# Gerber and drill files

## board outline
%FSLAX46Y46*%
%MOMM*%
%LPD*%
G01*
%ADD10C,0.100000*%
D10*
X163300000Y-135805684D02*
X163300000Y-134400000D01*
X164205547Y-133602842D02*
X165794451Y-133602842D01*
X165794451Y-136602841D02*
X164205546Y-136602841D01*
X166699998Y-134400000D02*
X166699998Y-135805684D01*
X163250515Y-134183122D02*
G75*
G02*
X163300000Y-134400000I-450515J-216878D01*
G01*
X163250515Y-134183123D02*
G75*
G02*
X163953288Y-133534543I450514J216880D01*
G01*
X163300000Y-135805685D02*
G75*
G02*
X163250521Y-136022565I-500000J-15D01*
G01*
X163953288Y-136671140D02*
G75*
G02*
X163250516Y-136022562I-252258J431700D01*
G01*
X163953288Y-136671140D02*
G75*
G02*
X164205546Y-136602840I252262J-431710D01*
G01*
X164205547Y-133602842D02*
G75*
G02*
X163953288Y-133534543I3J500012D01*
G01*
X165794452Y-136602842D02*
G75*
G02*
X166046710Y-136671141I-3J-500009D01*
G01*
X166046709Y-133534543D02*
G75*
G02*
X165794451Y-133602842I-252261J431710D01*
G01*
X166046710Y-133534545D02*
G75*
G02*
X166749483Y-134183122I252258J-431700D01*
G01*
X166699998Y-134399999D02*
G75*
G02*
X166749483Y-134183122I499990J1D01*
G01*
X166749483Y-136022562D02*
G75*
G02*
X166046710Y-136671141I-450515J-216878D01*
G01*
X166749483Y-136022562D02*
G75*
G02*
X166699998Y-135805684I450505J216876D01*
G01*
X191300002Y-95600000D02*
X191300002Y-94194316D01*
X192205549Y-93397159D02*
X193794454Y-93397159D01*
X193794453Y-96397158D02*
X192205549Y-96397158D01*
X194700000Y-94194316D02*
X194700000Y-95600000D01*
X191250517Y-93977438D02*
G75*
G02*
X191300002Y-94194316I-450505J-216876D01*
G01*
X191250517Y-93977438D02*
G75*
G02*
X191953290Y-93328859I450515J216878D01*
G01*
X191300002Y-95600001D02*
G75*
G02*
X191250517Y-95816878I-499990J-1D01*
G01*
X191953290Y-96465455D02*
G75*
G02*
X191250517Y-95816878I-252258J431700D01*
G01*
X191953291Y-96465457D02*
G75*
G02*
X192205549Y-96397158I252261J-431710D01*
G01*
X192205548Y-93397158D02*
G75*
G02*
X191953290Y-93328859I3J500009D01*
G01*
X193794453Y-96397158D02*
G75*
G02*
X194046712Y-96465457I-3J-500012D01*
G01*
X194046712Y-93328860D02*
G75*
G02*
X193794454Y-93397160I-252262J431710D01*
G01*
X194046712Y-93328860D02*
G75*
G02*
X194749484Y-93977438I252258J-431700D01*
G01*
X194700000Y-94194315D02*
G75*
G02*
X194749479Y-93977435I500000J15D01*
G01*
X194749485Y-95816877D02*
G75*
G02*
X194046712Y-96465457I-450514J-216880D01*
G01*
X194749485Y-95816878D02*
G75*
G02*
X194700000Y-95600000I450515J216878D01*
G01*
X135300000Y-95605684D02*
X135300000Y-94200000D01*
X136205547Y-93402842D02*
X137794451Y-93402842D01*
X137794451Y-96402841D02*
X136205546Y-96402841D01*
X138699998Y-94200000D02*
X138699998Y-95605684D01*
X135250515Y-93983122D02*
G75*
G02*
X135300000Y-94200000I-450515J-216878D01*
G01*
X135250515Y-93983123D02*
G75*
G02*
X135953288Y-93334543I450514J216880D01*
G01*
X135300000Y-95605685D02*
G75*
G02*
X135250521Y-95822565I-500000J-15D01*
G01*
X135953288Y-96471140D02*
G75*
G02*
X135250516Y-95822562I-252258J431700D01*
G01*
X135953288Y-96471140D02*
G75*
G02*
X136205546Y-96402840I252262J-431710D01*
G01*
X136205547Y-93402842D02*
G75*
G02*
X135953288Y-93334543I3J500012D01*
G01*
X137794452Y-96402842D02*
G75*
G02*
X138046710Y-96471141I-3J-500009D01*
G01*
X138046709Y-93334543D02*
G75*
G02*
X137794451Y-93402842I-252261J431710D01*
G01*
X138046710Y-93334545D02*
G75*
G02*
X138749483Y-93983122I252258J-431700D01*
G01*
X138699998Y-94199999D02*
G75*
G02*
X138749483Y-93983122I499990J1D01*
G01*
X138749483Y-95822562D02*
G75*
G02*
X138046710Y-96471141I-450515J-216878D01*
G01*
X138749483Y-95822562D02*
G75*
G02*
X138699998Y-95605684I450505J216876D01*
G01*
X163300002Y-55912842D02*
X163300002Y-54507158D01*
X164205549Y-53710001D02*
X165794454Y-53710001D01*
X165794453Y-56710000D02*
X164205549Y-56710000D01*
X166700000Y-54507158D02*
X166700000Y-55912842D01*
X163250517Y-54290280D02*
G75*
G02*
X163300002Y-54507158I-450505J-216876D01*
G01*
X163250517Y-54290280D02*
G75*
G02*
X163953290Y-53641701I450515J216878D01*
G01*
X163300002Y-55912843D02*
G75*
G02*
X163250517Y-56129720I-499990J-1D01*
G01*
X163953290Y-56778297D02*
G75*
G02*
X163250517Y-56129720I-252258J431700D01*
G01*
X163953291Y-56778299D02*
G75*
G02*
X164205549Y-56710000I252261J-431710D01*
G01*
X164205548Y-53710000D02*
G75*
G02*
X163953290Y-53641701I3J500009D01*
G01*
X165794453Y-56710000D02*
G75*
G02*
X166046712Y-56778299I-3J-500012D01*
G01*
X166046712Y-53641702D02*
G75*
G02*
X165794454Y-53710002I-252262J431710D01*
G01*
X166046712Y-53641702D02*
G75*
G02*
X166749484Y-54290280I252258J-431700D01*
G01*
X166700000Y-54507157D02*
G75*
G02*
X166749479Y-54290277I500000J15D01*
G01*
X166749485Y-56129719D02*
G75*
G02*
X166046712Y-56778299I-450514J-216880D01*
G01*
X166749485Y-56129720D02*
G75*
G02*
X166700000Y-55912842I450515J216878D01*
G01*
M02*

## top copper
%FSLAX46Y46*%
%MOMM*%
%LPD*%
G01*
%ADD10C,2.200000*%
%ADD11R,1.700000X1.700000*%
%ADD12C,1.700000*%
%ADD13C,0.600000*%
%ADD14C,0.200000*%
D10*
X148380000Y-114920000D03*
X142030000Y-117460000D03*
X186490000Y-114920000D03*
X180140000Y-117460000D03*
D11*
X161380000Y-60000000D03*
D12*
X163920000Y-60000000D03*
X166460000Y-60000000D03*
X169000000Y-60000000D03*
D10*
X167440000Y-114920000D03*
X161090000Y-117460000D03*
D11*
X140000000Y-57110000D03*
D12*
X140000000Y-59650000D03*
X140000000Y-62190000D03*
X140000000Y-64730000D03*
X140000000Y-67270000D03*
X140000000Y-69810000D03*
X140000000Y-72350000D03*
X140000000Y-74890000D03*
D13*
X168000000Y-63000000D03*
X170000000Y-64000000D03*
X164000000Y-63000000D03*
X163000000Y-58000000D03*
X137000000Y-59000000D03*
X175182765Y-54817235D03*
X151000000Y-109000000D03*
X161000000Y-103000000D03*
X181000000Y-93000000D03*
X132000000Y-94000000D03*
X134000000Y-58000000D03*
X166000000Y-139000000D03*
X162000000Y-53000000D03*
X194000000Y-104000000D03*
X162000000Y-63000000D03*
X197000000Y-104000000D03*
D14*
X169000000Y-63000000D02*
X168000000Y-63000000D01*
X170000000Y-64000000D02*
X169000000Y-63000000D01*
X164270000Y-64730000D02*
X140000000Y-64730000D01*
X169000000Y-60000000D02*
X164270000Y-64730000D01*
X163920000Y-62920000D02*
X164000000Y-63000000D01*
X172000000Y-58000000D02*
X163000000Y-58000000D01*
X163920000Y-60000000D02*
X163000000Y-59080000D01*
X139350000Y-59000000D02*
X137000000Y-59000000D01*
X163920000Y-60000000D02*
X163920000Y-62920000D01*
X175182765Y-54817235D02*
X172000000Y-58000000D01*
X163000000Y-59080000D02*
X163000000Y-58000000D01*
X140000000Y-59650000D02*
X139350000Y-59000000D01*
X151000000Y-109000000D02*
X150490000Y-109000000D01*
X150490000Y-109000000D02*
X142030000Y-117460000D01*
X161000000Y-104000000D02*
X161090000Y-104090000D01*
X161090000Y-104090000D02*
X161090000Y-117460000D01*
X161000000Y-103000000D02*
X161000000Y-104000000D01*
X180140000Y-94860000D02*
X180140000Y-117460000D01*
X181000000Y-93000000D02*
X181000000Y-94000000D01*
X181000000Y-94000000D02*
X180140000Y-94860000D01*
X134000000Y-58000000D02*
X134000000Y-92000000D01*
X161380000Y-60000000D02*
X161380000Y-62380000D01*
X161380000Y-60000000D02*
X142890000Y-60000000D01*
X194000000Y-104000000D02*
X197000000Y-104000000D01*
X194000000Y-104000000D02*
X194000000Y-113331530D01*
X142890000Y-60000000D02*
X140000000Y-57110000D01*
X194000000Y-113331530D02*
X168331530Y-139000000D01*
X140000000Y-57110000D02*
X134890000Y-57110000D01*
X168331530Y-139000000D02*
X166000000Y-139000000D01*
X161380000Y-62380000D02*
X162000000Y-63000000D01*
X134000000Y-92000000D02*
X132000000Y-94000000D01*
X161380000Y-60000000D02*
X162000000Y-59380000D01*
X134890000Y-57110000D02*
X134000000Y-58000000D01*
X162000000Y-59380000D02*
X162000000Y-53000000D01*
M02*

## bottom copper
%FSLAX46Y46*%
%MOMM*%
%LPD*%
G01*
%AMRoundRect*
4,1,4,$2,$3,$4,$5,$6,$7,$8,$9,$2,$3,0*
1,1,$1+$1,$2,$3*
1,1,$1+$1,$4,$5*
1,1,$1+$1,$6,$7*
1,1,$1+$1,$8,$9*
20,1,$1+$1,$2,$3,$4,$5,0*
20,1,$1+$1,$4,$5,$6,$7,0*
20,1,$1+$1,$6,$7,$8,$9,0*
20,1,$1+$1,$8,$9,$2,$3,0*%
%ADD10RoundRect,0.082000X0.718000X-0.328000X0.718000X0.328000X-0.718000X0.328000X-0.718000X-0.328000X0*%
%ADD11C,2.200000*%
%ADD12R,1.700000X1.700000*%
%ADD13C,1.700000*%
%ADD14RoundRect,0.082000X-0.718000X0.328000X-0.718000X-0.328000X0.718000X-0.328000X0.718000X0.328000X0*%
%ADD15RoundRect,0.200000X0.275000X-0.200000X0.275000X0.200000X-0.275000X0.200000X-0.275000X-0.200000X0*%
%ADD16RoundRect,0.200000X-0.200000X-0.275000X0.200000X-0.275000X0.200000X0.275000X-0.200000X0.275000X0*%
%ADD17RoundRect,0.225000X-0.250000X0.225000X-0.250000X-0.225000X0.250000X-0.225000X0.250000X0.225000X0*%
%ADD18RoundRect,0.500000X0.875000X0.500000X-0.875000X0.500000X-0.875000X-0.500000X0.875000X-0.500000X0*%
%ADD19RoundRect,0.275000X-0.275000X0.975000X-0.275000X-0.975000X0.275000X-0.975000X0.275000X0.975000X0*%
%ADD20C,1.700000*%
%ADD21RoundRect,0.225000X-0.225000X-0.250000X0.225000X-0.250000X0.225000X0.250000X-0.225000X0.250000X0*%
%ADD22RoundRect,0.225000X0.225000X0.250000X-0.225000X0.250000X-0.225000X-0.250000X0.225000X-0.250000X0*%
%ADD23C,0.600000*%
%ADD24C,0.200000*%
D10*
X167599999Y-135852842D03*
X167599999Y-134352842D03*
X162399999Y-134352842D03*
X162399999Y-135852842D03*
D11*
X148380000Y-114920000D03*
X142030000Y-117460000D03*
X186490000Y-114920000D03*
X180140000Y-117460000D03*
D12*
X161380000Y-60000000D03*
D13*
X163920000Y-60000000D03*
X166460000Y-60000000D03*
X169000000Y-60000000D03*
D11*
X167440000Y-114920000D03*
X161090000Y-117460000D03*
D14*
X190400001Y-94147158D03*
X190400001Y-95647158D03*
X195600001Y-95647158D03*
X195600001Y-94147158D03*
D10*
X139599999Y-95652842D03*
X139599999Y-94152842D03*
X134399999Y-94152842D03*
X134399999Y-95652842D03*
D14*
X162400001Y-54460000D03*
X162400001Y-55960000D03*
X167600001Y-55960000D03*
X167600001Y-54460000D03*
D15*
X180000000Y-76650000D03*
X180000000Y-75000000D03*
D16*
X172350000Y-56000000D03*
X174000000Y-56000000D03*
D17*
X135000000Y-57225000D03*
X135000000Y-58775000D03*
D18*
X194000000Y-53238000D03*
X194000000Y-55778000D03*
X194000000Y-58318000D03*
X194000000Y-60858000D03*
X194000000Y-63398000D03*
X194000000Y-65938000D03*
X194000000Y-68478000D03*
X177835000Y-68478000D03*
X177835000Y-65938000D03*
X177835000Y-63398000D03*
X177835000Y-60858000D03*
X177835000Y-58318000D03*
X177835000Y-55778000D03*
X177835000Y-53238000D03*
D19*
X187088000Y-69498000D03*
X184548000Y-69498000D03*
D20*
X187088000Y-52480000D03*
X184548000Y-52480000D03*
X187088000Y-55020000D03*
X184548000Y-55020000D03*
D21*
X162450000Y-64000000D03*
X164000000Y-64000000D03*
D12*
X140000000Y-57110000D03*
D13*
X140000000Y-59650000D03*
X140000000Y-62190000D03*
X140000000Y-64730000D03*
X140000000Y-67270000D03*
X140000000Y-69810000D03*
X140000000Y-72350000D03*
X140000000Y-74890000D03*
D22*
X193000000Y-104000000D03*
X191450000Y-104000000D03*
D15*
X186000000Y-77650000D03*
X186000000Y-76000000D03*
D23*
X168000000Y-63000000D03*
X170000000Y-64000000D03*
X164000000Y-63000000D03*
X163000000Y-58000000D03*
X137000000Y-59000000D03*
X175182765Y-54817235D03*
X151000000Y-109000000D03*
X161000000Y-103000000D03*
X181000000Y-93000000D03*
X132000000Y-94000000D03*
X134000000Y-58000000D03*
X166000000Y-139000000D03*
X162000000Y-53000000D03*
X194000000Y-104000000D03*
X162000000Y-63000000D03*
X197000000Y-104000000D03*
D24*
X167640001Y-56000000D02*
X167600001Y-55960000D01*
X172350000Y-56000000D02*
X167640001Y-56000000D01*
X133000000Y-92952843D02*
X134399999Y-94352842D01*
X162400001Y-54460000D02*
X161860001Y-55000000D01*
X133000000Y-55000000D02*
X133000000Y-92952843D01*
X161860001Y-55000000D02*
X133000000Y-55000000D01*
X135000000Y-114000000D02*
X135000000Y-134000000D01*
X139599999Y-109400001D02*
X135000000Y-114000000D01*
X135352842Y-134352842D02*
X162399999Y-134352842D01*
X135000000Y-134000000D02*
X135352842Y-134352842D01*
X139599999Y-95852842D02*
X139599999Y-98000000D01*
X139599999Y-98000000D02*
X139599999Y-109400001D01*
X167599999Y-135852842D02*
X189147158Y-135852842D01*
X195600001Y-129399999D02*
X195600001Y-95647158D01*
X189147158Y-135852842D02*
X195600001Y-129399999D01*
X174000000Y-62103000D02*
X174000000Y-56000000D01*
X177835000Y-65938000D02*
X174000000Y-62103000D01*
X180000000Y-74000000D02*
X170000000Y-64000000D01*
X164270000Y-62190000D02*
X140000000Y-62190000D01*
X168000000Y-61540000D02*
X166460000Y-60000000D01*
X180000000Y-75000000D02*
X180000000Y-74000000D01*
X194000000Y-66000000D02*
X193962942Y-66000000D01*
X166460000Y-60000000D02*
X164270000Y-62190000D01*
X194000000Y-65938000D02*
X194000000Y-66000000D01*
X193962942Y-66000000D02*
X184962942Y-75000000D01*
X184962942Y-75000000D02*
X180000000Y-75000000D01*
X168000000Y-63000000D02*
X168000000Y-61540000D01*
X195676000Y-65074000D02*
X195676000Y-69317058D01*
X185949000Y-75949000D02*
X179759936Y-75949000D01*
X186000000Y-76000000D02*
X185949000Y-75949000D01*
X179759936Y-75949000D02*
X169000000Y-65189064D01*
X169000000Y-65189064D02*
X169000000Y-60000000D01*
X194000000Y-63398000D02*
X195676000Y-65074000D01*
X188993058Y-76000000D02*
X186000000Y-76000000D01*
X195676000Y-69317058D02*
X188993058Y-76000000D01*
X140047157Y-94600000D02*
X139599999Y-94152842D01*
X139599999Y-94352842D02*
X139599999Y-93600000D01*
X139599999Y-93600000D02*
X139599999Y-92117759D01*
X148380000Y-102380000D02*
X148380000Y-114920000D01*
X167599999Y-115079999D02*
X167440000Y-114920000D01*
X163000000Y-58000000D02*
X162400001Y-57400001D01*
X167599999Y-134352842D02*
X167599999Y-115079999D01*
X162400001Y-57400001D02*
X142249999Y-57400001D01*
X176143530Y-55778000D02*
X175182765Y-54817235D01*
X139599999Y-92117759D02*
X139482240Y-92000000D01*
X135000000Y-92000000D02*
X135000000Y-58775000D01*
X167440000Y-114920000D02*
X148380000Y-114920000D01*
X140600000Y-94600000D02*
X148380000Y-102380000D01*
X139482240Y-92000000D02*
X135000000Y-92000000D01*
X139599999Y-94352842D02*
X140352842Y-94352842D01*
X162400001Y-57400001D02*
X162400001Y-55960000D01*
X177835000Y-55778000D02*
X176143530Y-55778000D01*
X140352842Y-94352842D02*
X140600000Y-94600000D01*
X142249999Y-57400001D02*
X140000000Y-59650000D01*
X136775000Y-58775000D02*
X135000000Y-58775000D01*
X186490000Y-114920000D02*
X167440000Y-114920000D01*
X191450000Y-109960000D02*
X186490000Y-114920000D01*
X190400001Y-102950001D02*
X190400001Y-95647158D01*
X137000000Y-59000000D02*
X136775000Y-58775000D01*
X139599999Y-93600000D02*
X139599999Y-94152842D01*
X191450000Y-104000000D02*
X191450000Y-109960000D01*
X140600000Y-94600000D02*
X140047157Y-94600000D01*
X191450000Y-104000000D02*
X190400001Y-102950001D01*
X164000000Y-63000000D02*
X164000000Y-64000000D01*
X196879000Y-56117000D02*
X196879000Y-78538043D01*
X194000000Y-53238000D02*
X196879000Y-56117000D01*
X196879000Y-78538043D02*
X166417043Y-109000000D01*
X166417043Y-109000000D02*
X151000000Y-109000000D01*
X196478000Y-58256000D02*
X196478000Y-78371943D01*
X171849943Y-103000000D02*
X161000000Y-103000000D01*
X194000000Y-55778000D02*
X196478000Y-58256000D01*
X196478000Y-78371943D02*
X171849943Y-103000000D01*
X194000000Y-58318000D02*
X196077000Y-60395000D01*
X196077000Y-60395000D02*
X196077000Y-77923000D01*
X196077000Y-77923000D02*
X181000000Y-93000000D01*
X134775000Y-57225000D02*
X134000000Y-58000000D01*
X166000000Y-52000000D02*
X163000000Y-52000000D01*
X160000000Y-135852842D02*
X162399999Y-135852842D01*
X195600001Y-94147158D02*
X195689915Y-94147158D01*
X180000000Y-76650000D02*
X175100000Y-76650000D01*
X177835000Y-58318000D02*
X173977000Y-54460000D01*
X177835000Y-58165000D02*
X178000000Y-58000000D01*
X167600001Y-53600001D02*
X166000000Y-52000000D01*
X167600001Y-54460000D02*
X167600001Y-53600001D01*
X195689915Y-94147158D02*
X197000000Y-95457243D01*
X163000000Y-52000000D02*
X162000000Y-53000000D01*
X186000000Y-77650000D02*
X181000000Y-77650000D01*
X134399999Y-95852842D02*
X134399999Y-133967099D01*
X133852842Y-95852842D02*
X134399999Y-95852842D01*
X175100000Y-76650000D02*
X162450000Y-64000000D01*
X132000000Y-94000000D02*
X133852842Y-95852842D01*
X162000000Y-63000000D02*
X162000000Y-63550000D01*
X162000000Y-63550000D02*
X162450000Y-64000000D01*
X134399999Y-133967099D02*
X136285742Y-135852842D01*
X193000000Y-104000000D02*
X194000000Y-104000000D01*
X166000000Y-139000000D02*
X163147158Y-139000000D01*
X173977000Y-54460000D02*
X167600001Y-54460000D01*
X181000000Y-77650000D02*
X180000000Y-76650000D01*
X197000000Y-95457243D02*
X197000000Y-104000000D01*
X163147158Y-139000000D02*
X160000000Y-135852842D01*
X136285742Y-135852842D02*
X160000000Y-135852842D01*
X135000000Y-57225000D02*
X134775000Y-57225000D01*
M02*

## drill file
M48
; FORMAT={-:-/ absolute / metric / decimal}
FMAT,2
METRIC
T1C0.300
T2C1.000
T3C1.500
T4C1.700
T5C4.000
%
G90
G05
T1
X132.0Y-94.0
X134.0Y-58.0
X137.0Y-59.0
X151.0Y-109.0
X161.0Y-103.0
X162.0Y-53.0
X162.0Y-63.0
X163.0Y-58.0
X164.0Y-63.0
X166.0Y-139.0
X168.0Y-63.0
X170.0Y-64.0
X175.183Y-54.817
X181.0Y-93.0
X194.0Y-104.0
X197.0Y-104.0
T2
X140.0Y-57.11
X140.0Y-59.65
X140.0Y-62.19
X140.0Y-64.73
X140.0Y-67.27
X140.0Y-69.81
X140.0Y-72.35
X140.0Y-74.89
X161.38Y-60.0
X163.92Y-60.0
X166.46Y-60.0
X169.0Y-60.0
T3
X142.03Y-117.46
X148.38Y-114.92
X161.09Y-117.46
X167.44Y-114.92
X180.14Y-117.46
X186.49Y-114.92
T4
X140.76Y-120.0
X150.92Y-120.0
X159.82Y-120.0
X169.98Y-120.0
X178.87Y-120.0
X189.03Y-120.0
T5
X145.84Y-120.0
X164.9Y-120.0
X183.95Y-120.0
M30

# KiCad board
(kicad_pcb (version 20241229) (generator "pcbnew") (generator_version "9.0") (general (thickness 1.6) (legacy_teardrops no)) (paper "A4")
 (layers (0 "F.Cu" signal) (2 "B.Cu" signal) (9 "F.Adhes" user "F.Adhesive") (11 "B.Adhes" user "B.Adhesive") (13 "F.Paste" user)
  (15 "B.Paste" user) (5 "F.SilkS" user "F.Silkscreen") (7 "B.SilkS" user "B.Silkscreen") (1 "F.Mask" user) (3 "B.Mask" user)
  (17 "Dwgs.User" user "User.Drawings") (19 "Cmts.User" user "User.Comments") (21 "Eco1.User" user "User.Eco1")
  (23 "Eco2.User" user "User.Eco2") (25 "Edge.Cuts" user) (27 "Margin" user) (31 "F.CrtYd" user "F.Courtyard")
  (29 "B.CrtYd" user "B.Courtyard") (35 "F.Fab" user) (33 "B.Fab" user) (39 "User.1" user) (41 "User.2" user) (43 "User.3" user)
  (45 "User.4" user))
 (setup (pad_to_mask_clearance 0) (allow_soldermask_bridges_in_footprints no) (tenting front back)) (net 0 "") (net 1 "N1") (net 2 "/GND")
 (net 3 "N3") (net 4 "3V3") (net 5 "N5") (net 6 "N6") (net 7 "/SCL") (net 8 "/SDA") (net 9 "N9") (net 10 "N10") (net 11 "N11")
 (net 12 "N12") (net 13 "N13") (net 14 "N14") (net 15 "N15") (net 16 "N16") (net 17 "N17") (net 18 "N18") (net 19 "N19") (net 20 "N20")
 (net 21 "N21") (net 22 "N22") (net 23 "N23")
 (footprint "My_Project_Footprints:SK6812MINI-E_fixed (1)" (layer "F.Cu") (at 165 135 180)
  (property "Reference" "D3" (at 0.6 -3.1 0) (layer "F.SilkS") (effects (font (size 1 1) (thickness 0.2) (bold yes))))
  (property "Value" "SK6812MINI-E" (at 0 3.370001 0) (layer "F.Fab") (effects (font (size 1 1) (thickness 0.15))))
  (fp_line (start 1.7 -0.805684) (end 1.7 0.6) (stroke (width 0.1) (type solid)) (layer "Edge.Cuts"))
  (fp_line (start 0.794453 1.397158) (end -0.794451 1.397158) (stroke (width 0.1) (type solid)) (layer "Edge.Cuts"))
  (fp_line (start -0.794451 -1.602841) (end 0.794454 -1.602841) (stroke (width 0.1) (type solid)) (layer "Edge.Cuts"))
  (fp_line (start -1.699998 0.6) (end -1.699998 -0.805684) (stroke (width 0.1) (type solid)) (layer "Edge.Cuts"))
  (fp_arc (start 1.749485 0.816878) (mid 1.712528 0.711226) (end 1.7 0.6) (stroke (width 0.1) (type solid)) (layer "Edge.Cuts"))
  (fp_arc (start 1.749485 0.816877) (mid 1.638073 1.401193) (end 1.046712 1.465457) (stroke (width 0.1) (type solid)) (layer "Edge.Cuts"))
  (fp_arc (start 1.7 -0.805685) (mid 1.712528 -0.91691) (end 1.749485 -1.022562) (stroke (width 0.1) (type solid)) (layer "Edge.Cuts"))
  (fp_arc (start 1.046712 -1.67114) (mid 1.638072 -1.606876) (end 1.749485 -1.022562) (stroke (width 0.1) (type solid)) (layer "Edge.Cuts"))
  (fp_arc (start 1.046712 -1.67114) (mid 0.925124 -1.620218) (end 0.794454 -1.602841) (stroke (width 0.1) (type solid)) (layer "Edge.Cuts"))
  (fp_arc (start 0.794453 1.397158) (mid 0.925124 1.414535) (end 1.046712 1.465457) (stroke (width 0.1) (type solid)) (layer "Edge.Cuts"))
  (fp_arc (start -0.794452 -1.602842) (mid -0.925122 -1.620219) (end -1.04671 -1.671141) (stroke (width 0.1) (type solid))
   (layer "Edge.Cuts"))
  (fp_arc (start -1.046709 1.465457) (mid -0.925121 1.414535) (end -0.794451 1.397158) (stroke (width 0.1) (type solid)) (layer "Edge.Cuts"))
  (fp_arc (start -1.04671 1.465455) (mid -1.638069 1.401192) (end -1.749483 0.816878) (stroke (width 0.1) (type solid)) (layer "Edge.Cuts"))
  (fp_arc (start -1.699998 0.600001) (mid -1.712526 0.711226) (end -1.749483 0.816878) (stroke (width 0.1) (type solid)) (layer "Edge.Cuts"))
  (fp_arc (start -1.749483 -1.022562) (mid -1.63807 -1.606877) (end -1.04671 -1.671141) (stroke (width 0.1) (type solid))
   (layer "Edge.Cuts"))
  (fp_arc (start -1.749483 -1.022562) (mid -1.712526 -0.91691) (end -1.699998 -0.805684) (stroke (width 0.1) (type solid))
   (layer "Edge.Cuts"))
  (pad "1" smd roundrect (at -2.599999 -0.852842 90) (size 0.82 1.6) (layers "B.Cu" "B.Mask" "B.Paste") (roundrect_rratio 0.1) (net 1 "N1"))
  (pad "2" smd roundrect (at -2.599999 0.647158 90) (size 0.82 1.6) (layers "B.Cu" "B.Mask" "B.Paste") (roundrect_rratio 0.1) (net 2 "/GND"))
  (pad "3" smd roundrect (at 2.600001 0.647158 90) (size 0.82 1.6) (layers "B.Cu" "B.Mask" "B.Paste") (roundrect_rratio 0.1) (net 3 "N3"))
  (pad "4" smd roundrect (at 2.600001 -0.852842 90) (size 0.82 1.6) (layers "B.Cu" "B.Mask" "B.Paste") (roundrect_rratio 0.1) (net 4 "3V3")))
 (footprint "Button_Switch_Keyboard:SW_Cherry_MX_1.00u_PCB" (layer "F.Cu") (at 148.38 114.92)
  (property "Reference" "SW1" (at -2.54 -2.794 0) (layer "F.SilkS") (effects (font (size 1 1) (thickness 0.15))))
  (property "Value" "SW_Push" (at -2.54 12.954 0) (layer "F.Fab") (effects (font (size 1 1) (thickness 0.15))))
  (pad "" np_thru_hole circle (at -7.62 5.08) (size 1.7 1.7) (drill 1.7) (layers "*.Cu" "*.Mask"))
  (pad "" np_thru_hole circle (at -2.54 5.08) (size 4 4) (drill 4) (layers "*.Cu" "*.Mask"))
  (pad "" np_thru_hole circle (at 2.54 5.08) (size 1.7 1.7) (drill 1.7) (layers "*.Cu" "*.Mask"))
  (pad "1" thru_hole circle (at 0 0) (size 2.2 2.2) (drill 1.5) (layers "*.Cu" "*.Mask") (remove_unused_layers no) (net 2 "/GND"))
  (pad "2" thru_hole circle (at -6.35 2.54) (size 2.2 2.2) (drill 1.5) (layers "*.Cu" "*.Mask") (remove_unused_layers no) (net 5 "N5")))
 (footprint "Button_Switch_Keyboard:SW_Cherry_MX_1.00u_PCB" (layer "F.Cu") (at 186.49 114.92)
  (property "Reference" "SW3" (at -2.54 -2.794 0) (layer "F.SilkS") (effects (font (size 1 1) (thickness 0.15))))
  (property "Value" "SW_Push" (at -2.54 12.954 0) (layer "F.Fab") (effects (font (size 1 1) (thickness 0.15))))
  (pad "" np_thru_hole circle (at -7.62 5.08) (size 1.7 1.7) (drill 1.7) (layers "*.Cu" "*.Mask"))
  (pad "" np_thru_hole circle (at -2.54 5.08) (size 4 4) (drill 4) (layers "*.Cu" "*.Mask"))
  (pad "" np_thru_hole circle (at 2.54 5.08) (size 1.7 1.7) (drill 1.7) (layers "*.Cu" "*.Mask"))
  (pad "1" thru_hole circle (at 0 0) (size 2.2 2.2) (drill 1.5) (layers "*.Cu" "*.Mask") (remove_unused_layers no) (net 2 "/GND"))
  (pad "2" thru_hole circle (at -6.35 2.54) (size 2.2 2.2) (drill 1.5) (layers "*.Cu" "*.Mask") (remove_unused_layers no) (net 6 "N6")))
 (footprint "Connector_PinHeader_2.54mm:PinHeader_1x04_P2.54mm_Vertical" (layer "F.Cu") (at 161.38 60 90)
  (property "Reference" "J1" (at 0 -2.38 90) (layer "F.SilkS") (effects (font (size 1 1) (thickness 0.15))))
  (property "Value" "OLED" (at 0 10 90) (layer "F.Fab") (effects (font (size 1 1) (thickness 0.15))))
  (pad "1" thru_hole rect (at 0 0 90) (size 1.7 1.7) (drill 1) (layers "*.Cu" "*.Mask") (remove_unused_layers no) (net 4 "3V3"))
  (pad "2" thru_hole circle (at 0 2.54 90) (size 1.7 1.7) (drill 1) (layers "*.Cu" "*.Mask") (remove_unused_layers no) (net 2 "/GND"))
  (pad "3" thru_hole circle (at 0 5.08 90) (size 1.7 1.7) (drill 1) (layers "*.Cu" "*.Mask") (remove_unused_layers no) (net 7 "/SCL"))
  (pad "4" thru_hole circle (at 0 7.62 90) (size 1.7 1.7) (drill 1) (layers "*.Cu" "*.Mask") (remove_unused_layers no) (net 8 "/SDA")))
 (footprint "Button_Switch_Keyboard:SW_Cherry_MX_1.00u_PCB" (layer "F.Cu") (at 167.44 114.92)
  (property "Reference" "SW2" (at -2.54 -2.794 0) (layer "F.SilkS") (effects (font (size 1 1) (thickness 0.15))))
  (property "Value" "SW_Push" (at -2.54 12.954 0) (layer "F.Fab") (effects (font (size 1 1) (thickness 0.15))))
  (pad "" np_thru_hole circle (at -7.62 5.08) (size 1.7 1.7) (drill 1.7) (layers "*.Cu" "*.Mask"))
  (pad "" np_thru_hole circle (at -2.54 5.08) (size 4 4) (drill 4) (layers "*.Cu" "*.Mask"))
  (pad "" np_thru_hole circle (at 2.54 5.08) (size 1.7 1.7) (drill 1.7) (layers "*.Cu" "*.Mask"))
  (pad "1" thru_hole circle (at 0 0) (size 2.2 2.2) (drill 1.5) (layers "*.Cu" "*.Mask") (remove_unused_layers no) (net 2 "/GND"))
  (pad "2" thru_hole circle (at -6.35 2.54) (size 2.2 2.2) (drill 1.5) (layers "*.Cu" "*.Mask") (remove_unused_layers no) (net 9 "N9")))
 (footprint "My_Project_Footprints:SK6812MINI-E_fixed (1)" (layer "F.Cu") (at 193 95)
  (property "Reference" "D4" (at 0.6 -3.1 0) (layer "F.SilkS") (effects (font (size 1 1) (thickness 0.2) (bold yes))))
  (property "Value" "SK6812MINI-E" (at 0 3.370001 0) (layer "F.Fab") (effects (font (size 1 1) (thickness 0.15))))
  (fp_line (start -1.699998 0.6) (end -1.699998 -0.805684) (stroke (width 0.1) (type solid)) (layer "Edge.Cuts"))
  (fp_line (start -0.794451 -1.602841) (end 0.794454 -1.602841) (stroke (width 0.1) (type solid)) (layer "Edge.Cuts"))
  (fp_line (start 0.794453 1.397158) (end -0.794451 1.397158) (stroke (width 0.1) (type solid)) (layer "Edge.Cuts"))
  (fp_line (start 1.7 -0.805684) (end 1.7 0.6) (stroke (width 0.1) (type solid)) (layer "Edge.Cuts"))
  (fp_arc (start -1.749483 -1.022562) (mid -1.712526 -0.91691) (end -1.699998 -0.805684) (stroke (width 0.1) (type solid))
   (layer "Edge.Cuts"))
  (fp_arc (start -1.749483 -1.022562) (mid -1.63807 -1.606877) (end -1.04671 -1.671141) (stroke (width 0.1) (type solid))
   (layer "Edge.Cuts"))
  (fp_arc (start -1.699998 0.600001) (mid -1.712526 0.711226) (end -1.749483 0.816878) (stroke (width 0.1) (type solid)) (layer "Edge.Cuts"))
  (fp_arc (start -1.04671 1.465455) (mid -1.638069 1.401192) (end -1.749483 0.816878) (stroke (width 0.1) (type solid)) (layer "Edge.Cuts"))
  (fp_arc (start -1.046709 1.465457) (mid -0.925121 1.414535) (end -0.794451 1.397158) (stroke (width 0.1) (type solid)) (layer "Edge.Cuts"))
  (fp_arc (start -0.794452 -1.602842) (mid -0.925122 -1.620219) (end -1.04671 -1.671141) (stroke (width 0.1) (type solid))
   (layer "Edge.Cuts"))
  (fp_arc (start 0.794453 1.397158) (mid 0.925124 1.414535) (end 1.046712 1.465457) (stroke (width 0.1) (type solid)) (layer "Edge.Cuts"))
  (fp_arc (start 1.046712 -1.67114) (mid 0.925124 -1.620218) (end 0.794454 -1.602841) (stroke (width 0.1) (type solid)) (layer "Edge.Cuts"))
  (fp_arc (start 1.046712 -1.67114) (mid 1.638072 -1.606876) (end 1.749485 -1.022562) (stroke (width 0.1) (type solid)) (layer "Edge.Cuts"))
  (fp_arc (start 1.7 -0.805685) (mid 1.712528 -0.91691) (end 1.749485 -1.022562) (stroke (width 0.1) (type solid)) (layer "Edge.Cuts"))
  (fp_arc (start 1.749485 0.816877) (mid 1.638073 1.401193) (end 1.046712 1.465457) (stroke (width 0.1) (type solid)) (layer "Edge.Cuts"))
  (fp_arc (start 1.749485 0.816878) (mid 1.712528 0.711226) (end 1.7 0.6) (stroke (width 0.1) (type solid)) (layer "Edge.Cuts"))
  (pad "1" smd roundrect (at -2.599999 -0.852842 270) (size 0.82 1.6) (layers "B.Cu" "B.Mask" "B.Paste") (roundrect_rratio 0.1)
   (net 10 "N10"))
  (pad "2" smd roundrect (at -2.599999 0.647158 270) (size 0.82 1.6) (layers "B.Cu" "B.Mask" "B.Paste") (roundrect_rratio 0.1)
   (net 2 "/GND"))
  (pad "3" smd roundrect (at 2.600001 0.647158 270) (size 0.82 1.6) (layers "B.Cu" "B.Mask" "B.Paste") (roundrect_rratio 0.1) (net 1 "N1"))
  (pad "4" smd roundrect (at 2.600001 -0.852842 270) (size 0.82 1.6) (layers "B.Cu" "B.Mask" "B.Paste") (roundrect_rratio 0.1) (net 4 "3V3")))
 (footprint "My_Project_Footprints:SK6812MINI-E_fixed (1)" (layer "F.Cu") (at 137 94.8 180)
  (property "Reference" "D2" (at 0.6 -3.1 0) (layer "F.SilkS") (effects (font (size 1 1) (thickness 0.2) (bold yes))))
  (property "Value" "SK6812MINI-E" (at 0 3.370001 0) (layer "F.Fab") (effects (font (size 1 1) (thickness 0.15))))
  (fp_line (start 1.7 -0.805684) (end 1.7 0.6) (stroke (width 0.1) (type solid)) (layer "Edge.Cuts"))
  (fp_line (start 0.794453 1.397158) (end -0.794451 1.397158) (stroke (width 0.1) (type solid)) (layer "Edge.Cuts"))
  (fp_line (start -0.794451 -1.602841) (end 0.794454 -1.602841) (stroke (width 0.1) (type solid)) (layer "Edge.Cuts"))
  (fp_line (start -1.699998 0.6) (end -1.699998 -0.805684) (stroke (width 0.1) (type solid)) (layer "Edge.Cuts"))
  (fp_arc (start 1.749485 0.816878) (mid 1.712528 0.711226) (end 1.7 0.6) (stroke (width 0.1) (type solid)) (layer "Edge.Cuts"))
  (fp_arc (start 1.749485 0.816877) (mid 1.638073 1.401193) (end 1.046712 1.465457) (stroke (width 0.1) (type solid)) (layer "Edge.Cuts"))
  (fp_arc (start 1.7 -0.805685) (mid 1.712528 -0.91691) (end 1.749485 -1.022562) (stroke (width 0.1) (type solid)) (layer "Edge.Cuts"))
  (fp_arc (start 1.046712 -1.67114) (mid 1.638072 -1.606876) (end 1.749485 -1.022562) (stroke (width 0.1) (type solid)) (layer "Edge.Cuts"))
  (fp_arc (start 1.046712 -1.67114) (mid 0.925124 -1.620218) (end 0.794454 -1.602841) (stroke (width 0.1) (type solid)) (layer "Edge.Cuts"))
  (fp_arc (start 0.794453 1.397158) (mid 0.925124 1.414535) (end 1.046712 1.465457) (stroke (width 0.1) (type solid)) (layer "Edge.Cuts"))
  (fp_arc (start -0.794452 -1.602842) (mid -0.925122 -1.620219) (end -1.04671 -1.671141) (stroke (width 0.1) (type solid))
   (layer "Edge.Cuts"))
  (fp_arc (start -1.046709 1.465457) (mid -0.925121 1.414535) (end -0.794451 1.397158) (stroke (width 0.1) (type solid)) (layer "Edge.Cuts"))
  (fp_arc (start -1.04671 1.465455) (mid -1.638069 1.401192) (end -1.749483 0.816878) (stroke (width 0.1) (type solid)) (layer "Edge.Cuts"))
  (fp_arc (start -1.699998 0.600001) (mid -1.712526 0.711226) (end -1.749483 0.816878) (stroke (width 0.1) (type solid)) (layer "Edge.Cuts"))
  (fp_arc (start -1.749483 -1.022562) (mid -1.63807 -1.606877) (end -1.04671 -1.671141) (stroke (width 0.1) (type solid))
   (layer "Edge.Cuts"))
  (fp_arc (start -1.749483 -1.022562) (mid -1.712526 -0.91691) (end -1.699998 -0.805684) (stroke (width 0.1) (type solid))
   (layer "Edge.Cuts"))
  (pad "1" smd roundrect (at -2.599999 -0.852842 90) (size 0.82 1.6) (layers "B.Cu" "B.Mask" "B.Paste") (roundrect_rratio 0.1) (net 3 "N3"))
  (pad "2" smd roundrect (at -2.599999 0.647158 90) (size 0.82 1.6) (layers "B.Cu" "B.Mask" "B.Paste") (roundrect_rratio 0.1) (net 2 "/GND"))
  (pad "3" smd roundrect (at 2.600001 0.647158 90) (size 0.82 1.6) (layers "B.Cu" "B.Mask" "B.Paste") (roundrect_rratio 0.1) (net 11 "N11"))
  (pad "4" smd roundrect (at 2.600001 -0.852842 90) (size 0.82 1.6) (layers "B.Cu" "B.Mask" "B.Paste") (roundrect_rratio 0.1) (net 4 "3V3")))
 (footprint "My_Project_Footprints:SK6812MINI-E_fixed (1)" (layer "F.Cu") (at 165 55.312842)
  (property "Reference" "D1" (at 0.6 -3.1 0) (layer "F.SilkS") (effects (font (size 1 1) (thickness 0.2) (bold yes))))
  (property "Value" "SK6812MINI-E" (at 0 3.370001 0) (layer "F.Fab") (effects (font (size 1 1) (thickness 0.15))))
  (fp_line (start -1.699998 0.6) (end -1.699998 -0.805684) (stroke (width 0.1) (type solid)) (layer "Edge.Cuts"))
  (fp_line (start -0.794451 -1.602841) (end 0.794454 -1.602841) (stroke (width 0.1) (type solid)) (layer "Edge.Cuts"))
  (fp_line (start 0.794453 1.397158) (end -0.794451 1.397158) (stroke (width 0.1) (type solid)) (layer "Edge.Cuts"))
  (fp_line (start 1.7 -0.805684) (end 1.7 0.6) (stroke (width 0.1) (type solid)) (layer "Edge.Cuts"))
  (fp_arc (start -1.749483 -1.022562) (mid -1.712526 -0.91691) (end -1.699998 -0.805684) (stroke (width 0.1) (type solid))
   (layer "Edge.Cuts"))
  (fp_arc (start -1.749483 -1.022562) (mid -1.63807 -1.606877) (end -1.04671 -1.671141) (stroke (width 0.1) (type solid))
   (layer "Edge.Cuts"))
  (fp_arc (start -1.699998 0.600001) (mid -1.712526 0.711226) (end -1.749483 0.816878) (stroke (width 0.1) (type solid)) (layer "Edge.Cuts"))
  (fp_arc (start -1.04671 1.465455) (mid -1.638069 1.401192) (end -1.749483 0.816878) (stroke (width 0.1) (type solid)) (layer "Edge.Cuts"))
  (fp_arc (start -1.046709 1.465457) (mid -0.925121 1.414535) (end -0.794451 1.397158) (stroke (width 0.1) (type solid)) (layer "Edge.Cuts"))
  (fp_arc (start -0.794452 -1.602842) (mid -0.925122 -1.620219) (end -1.04671 -1.671141) (stroke (width 0.1) (type solid))
   (layer "Edge.Cuts"))
  (fp_arc (start 0.794453 1.397158) (mid 0.925124 1.414535) (end 1.046712 1.465457) (stroke (width 0.1) (type solid)) (layer "Edge.Cuts"))
  (fp_arc (start 1.046712 -1.67114) (mid 0.925124 -1.620218) (end 0.794454 -1.602841) (stroke (width 0.1) (type solid)) (layer "Edge.Cuts"))
  (fp_arc (start 1.046712 -1.67114) (mid 1.638072 -1.606876) (end 1.749485 -1.022562) (stroke (width 0.1) (type solid)) (layer "Edge.Cuts"))
  (fp_arc (start 1.7 -0.805685) (mid 1.712528 -0.91691) (end 1.749485 -1.022562) (stroke (width 0.1) (type solid)) (layer "Edge.Cuts"))
  (fp_arc (start 1.749485 0.816877) (mid 1.638073 1.401193) (end 1.046712 1.465457) (stroke (width 0.1) (type solid)) (layer "Edge.Cuts"))
  (fp_arc (start 1.749485 0.816878) (mid 1.712528 0.711226) (end 1.7 0.6) (stroke (width 0.1) (type solid)) (layer "Edge.Cuts"))
  (pad "1" smd roundrect (at -2.599999 -0.852842 270) (size 0.82 1.6) (layers "B.Cu" "B.Mask" "B.Paste") (roundrect_rratio 0.1)
   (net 11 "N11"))
  (pad "2" smd roundrect (at -2.599999 0.647158 270) (size 0.82 1.6) (layers "B.Cu" "B.Mask" "B.Paste") (roundrect_rratio 0.1)
   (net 2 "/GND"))
  (pad "3" smd roundrect (at 2.600001 0.647158 270) (size 0.82 1.6) (layers "B.Cu" "B.Mask" "B.Paste") (roundrect_rratio 0.1) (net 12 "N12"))
  (pad "4" smd roundrect (at 2.600001 -0.852842 270) (size 0.82 1.6) (layers "B.Cu" "B.Mask" "B.Paste") (roundrect_rratio 0.1) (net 4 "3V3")))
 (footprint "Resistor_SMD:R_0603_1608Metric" (layer "B.Cu") (at 180 75.825 90)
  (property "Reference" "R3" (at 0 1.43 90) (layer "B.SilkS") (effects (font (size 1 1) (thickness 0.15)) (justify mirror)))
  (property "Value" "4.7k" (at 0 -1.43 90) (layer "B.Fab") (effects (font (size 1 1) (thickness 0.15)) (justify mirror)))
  (pad "1" smd roundrect (at -0.825 0 90) (size 0.8 0.95) (layers "B.Cu" "B.Mask" "B.Paste") (roundrect_rratio 0.25) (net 4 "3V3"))
  (pad "2" smd roundrect (at 0.825 0 90) (size 0.8 0.95) (layers "B.Cu" "B.Mask" "B.Paste") (roundrect_rratio 0.25) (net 7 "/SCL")))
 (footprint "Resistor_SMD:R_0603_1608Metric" (layer "B.Cu") (at 173.175 56)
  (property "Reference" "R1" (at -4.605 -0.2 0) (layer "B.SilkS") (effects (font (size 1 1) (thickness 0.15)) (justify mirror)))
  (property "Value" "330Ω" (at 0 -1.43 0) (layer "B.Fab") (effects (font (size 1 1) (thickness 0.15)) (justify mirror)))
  (pad "1" smd roundrect (at -0.825 0) (size 0.8 0.95) (layers "B.Cu" "B.Mask" "B.Paste") (roundrect_rratio 0.25) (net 12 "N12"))
  (pad "2" smd roundrect (at 0.825 0) (size 0.8 0.95) (layers "B.Cu" "B.Mask" "B.Paste") (roundrect_rratio 0.25) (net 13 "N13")))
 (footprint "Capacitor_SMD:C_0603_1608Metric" (layer "B.Cu") (at 135 58 -90)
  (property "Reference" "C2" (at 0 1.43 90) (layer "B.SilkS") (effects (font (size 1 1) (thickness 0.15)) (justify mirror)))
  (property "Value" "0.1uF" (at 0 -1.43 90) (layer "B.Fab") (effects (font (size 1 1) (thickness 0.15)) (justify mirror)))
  (pad "1" smd roundrect (at -0.775 0 270) (size 0.9 0.95) (layers "B.Cu" "B.Mask" "B.Paste") (roundrect_rratio 0.25) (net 4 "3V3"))
  (pad "2" smd roundrect (at 0.775 0 270) (size 0.9 0.95) (layers "B.Cu" "B.Mask" "B.Paste") (roundrect_rratio 0.25) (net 2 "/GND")))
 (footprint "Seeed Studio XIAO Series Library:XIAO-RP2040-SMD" (layer "B.Cu") (at 186 60.858 180)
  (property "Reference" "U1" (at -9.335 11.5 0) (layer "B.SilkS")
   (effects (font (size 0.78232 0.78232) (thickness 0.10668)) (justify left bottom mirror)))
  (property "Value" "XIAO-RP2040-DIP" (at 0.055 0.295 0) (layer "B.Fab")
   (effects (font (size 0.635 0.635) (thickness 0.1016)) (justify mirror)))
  (pad "1" smd roundrect (at -8 7.62 180) (size 2.75 2) (layers "B.Cu" "B.Mask" "B.Paste") (roundrect_rratio 0.25) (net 5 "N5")
   (solder_mask_margin 0.0508) (thermal_bridge_angle 45))
  (pad "2" smd roundrect (at -8 5.08 180) (size 2.75 2) (layers "B.Cu" "B.Mask" "B.Paste") (roundrect_rratio 0.25) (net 9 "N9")
   (solder_mask_margin 0.0508) (thermal_bridge_angle 45))
  (pad "3" smd roundrect (at -8 2.54 180) (size 2.75 2) (layers "B.Cu" "B.Mask" "B.Paste") (roundrect_rratio 0.25) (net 6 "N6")
   (solder_mask_margin 0.0508) (thermal_bridge_angle 45))
  (pad "4" smd roundrect (at -8 0 180) (size 2.75 2) (layers "B.Cu" "B.Mask" "B.Paste") (roundrect_rratio 0.25) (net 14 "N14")
   (solder_mask_margin 0.0508) (thermal_bridge_angle 45))
  (pad "5" smd roundrect (at -8 -2.54 180) (size 2.75 2) (layers "B.Cu" "B.Mask" "B.Paste") (roundrect_rratio 0.25) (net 8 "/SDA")
   (solder_mask_margin 0.0508) (thermal_bridge_angle 45))
  (pad "6" smd roundrect (at -8 -5.08 180) (size 2.75 2) (layers "B.Cu" "B.Mask" "B.Paste") (roundrect_rratio 0.25) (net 7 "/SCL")
   (solder_mask_margin 0.0508) (thermal_bridge_angle 45))
  (pad "7" smd roundrect (at -8 -7.62 180) (size 2.75 2) (layers "B.Cu" "B.Mask" "B.Paste") (roundrect_rratio 0.25) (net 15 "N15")
   (solder_mask_margin 0.0508) (thermal_bridge_angle 45))
  (pad "8" smd roundrect (at 8.165 -7.62 180) (size 2.75 2) (layers "B.Cu" "B.Mask" "B.Paste") (roundrect_rratio 0.25) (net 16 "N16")
   (solder_mask_margin 0.0508) (thermal_bridge_angle 45))
  (pad "9" smd roundrect (at 8.165 -5.08 180) (size 2.75 2) (layers "B.Cu" "B.Mask" "B.Paste") (roundrect_rratio 0.25) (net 13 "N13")
   (solder_mask_margin 0.0508) (thermal_bridge_angle 45))
  (pad "10" smd roundrect (at 8.165 -2.54 180) (size 2.75 2) (layers "B.Cu" "B.Mask" "B.Paste") (roundrect_rratio 0.25) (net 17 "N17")
   (solder_mask_margin 0.0508) (thermal_bridge_angle 45))
  (pad "11" smd roundrect (at 8.165 0 180) (size 2.75 2) (layers "B.Cu" "B.Mask" "B.Paste") (roundrect_rratio 0.25) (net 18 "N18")
   (solder_mask_margin 0.0508) (thermal_bridge_angle 45))
  (pad "12" smd roundrect (at 8.165 2.54 180) (size 2.75 2) (layers "B.Cu" "B.Mask" "B.Paste") (roundrect_rratio 0.25) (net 4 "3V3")
   (solder_mask_margin 0.0508) (thermal_bridge_angle 45))
  (pad "13" smd roundrect (at 8.165 5.08 180) (size 2.75 2) (layers "B.Cu" "B.Mask" "B.Paste") (roundrect_rratio 0.25) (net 2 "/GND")
   (solder_mask_margin 0.0508) (thermal_bridge_angle 45))
  (pad "14" smd roundrect (at 8.165 7.62 180) (size 2.75 2) (layers "B.Cu" "B.Mask" "B.Paste") (roundrect_rratio 0.25) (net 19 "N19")
   (solder_mask_margin 0.0508) (thermal_bridge_angle 45))
  (pad "15" smd roundrect (at -1.088 -8.64 270) (size 2.5 1.1) (layers "B.Cu" "B.Mask" "B.Paste") (roundrect_rratio 0.25)
   (thermal_bridge_angle 45))
  (pad "16" smd roundrect (at 1.452 -8.64 270) (size 2.5 1.1) (layers "B.Cu" "B.Mask" "B.Paste") (roundrect_rratio 0.25)
   (thermal_bridge_angle 45))
  (pad "17" smd circle (at -1.088 8.378 180) (size 1.7 1.7) (layers "B.Cu" "B.Mask" "B.Paste"))
  (pad "18" smd circle (at 1.452 8.378 180) (size 1.7 1.7) (layers "B.Cu" "B.Mask" "B.Paste"))
  (pad "19" smd circle (at -1.088 5.838 180) (size 1.7 1.7) (layers "B.Cu" "B.Mask" "B.Paste"))
  (pad "20" smd circle (at 1.452 5.838 180) (size 1.7 1.7) (layers "B.Cu" "B.Mask" "B.Paste")))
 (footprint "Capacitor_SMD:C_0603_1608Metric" (layer "B.Cu") (at 163.225 64)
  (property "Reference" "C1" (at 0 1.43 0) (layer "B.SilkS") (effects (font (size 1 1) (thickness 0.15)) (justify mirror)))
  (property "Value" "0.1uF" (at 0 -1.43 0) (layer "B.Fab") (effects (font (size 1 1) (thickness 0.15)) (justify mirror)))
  (pad "1" smd roundrect (at -0.775 0) (size 0.9 0.95) (layers "B.Cu" "B.Mask" "B.Paste") (roundrect_rratio 0.25) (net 4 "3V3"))
  (pad "2" smd roundrect (at 0.775 0) (size 0.9 0.95) (layers "B.Cu" "B.Mask" "B.Paste") (roundrect_rratio 0.25) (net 2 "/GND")))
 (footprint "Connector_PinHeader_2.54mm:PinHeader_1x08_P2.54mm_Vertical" (layer "B.Cu") (at 140 57.11 180)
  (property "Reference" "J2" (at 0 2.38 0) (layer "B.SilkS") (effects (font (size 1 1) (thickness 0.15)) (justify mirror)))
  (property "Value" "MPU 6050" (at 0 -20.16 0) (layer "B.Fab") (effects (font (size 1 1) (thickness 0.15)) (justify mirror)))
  (pad "1" thru_hole rect (at 0 0 180) (size 1.7 1.7) (drill 1) (layers "*.Cu" "*.Mask") (remove_unused_layers no) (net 4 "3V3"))
  (pad "2" thru_hole circle (at 0 -2.54 180) (size 1.7 1.7) (drill 1) (layers "*.Cu" "*.Mask") (remove_unused_layers no) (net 2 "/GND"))
  (pad "3" thru_hole circle (at 0 -5.08 180) (size 1.7 1.7) (drill 1) (layers "*.Cu" "*.Mask") (remove_unused_layers no) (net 7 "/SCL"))
  (pad "4" thru_hole circle (at 0 -7.62 180) (size 1.7 1.7) (drill 1) (layers "*.Cu" "*.Mask") (remove_unused_layers no) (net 8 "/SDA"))
  (pad "5" thru_hole circle (at 0 -10.16 180) (size 1.7 1.7) (drill 1) (layers "*.Cu" "*.Mask") (remove_unused_layers no) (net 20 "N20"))
  (pad "6" thru_hole circle (at 0 -12.7 180) (size 1.7 1.7) (drill 1) (layers "*.Cu" "*.Mask") (remove_unused_layers no) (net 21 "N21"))
  (pad "7" thru_hole circle (at 0 -15.24 180) (size 1.7 1.7) (drill 1) (layers "*.Cu" "*.Mask") (remove_unused_layers no) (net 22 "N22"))
  (pad "8" thru_hole circle (at 0 -17.78 180) (size 1.7 1.7) (drill 1) (layers "*.Cu" "*.Mask") (remove_unused_layers no) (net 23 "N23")))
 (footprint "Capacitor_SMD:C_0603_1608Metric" (layer "B.Cu") (at 192.225 104 180)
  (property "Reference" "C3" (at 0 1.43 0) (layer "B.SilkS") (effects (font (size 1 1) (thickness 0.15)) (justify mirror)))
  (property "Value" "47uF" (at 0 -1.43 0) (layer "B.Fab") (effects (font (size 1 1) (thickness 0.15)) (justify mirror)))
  (pad "1" smd roundrect (at -0.775 0 180) (size 0.9 0.95) (layers "B.Cu" "B.Mask" "B.Paste") (roundrect_rratio 0.25) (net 4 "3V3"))
  (pad "2" smd roundrect (at 0.775 0 180) (size 0.9 0.95) (layers "B.Cu" "B.Mask" "B.Paste") (roundrect_rratio 0.25) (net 2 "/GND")))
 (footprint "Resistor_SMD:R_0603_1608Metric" (layer "B.Cu") (at 186 76.825 90)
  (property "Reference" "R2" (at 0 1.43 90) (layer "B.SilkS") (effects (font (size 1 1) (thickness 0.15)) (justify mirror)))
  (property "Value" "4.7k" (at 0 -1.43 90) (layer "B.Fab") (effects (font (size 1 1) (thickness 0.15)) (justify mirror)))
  (pad "1" smd roundrect (at -0.825 0 90) (size 0.8 0.95) (layers "B.Cu" "B.Mask" "B.Paste") (roundrect_rratio 0.25) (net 4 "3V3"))
  (pad "2" smd roundrect (at 0.825 0 90) (size 0.8 0.95) (layers "B.Cu" "B.Mask" "B.Paste") (roundrect_rratio 0.25) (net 8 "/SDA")))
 (segment (start 167.640001 56) (end 167.600001 55.96) (width 0.2) (layer "B.Cu") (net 12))
 (segment (start 172.35 56) (end 167.640001 56) (width 0.2) (layer "B.Cu") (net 12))
 (segment (start 133 92.952843) (end 134.399999 94.352842) (width 0.2) (layer "B.Cu") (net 11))
 (segment (start 162.400001 54.46) (end 161.860001 55) (width 0.2) (layer "B.Cu") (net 11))
 (segment (start 133 55) (end 133 92.952843) (width 0.2) (layer "B.Cu") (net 11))
 (segment (start 161.860001 55) (end 133 55) (width 0.2) (layer "B.Cu") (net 11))
 (segment (start 135 114) (end 135 134) (width 0.2) (layer "B.Cu") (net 3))
 (segment (start 139.599999 109.400001) (end 135 114) (width 0.2) (layer "B.Cu") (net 3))
 (segment (start 135.352842 134.352842) (end 162.399999 134.352842) (width 0.2) (layer "B.Cu") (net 3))
 (segment (start 135 134) (end 135.352842 134.352842) (width 0.2) (layer "B.Cu") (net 3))
 (segment (start 139.599999 95.852842) (end 139.599999 98) (width 0.2) (layer "B.Cu") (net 3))
 (segment (start 139.599999 98) (end 139.599999 109.400001) (width 0.2) (layer "B.Cu") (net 3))
 (segment (start 167.599999 135.852842) (end 189.147158 135.852842) (width 0.2) (layer "B.Cu") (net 1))
 (segment (start 195.600001 129.399999) (end 195.600001 95.647158) (width 0.2) (layer "B.Cu") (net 1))
 (segment (start 189.147158 135.852842) (end 195.600001 129.399999) (width 0.2) (layer "B.Cu") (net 1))
 (segment (start 174 62.103) (end 174 56) (width 0.2) (layer "B.Cu") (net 13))
 (segment (start 177.835 65.938) (end 174 62.103) (width 0.2) (layer "B.Cu") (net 13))
 (segment (start 169 63) (end 168 63) (width 0.2) (layer "F.Cu") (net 7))
 (segment (start 170 64) (end 169 63) (width 0.2) (layer "F.Cu") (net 7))
 (via (at 168 63) (size 0.6) (drill 0.3) (layers "F.Cu" "B.Cu") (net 7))
 (via (at 170 64) (size 0.6) (drill 0.3) (layers "F.Cu" "B.Cu") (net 7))
 (segment (start 180 74) (end 170 64) (width 0.2) (layer "B.Cu") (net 7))
 (segment (start 164.27 62.19) (end 140 62.19) (width 0.2) (layer "B.Cu") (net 7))
 (segment (start 168 61.54) (end 166.46 60) (width 0.2) (layer "B.Cu") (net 7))
 (segment (start 180 75) (end 180 74) (width 0.2) (layer "B.Cu") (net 7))
 (segment (start 194 66) (end 193.962942 66) (width 0.2) (layer "B.Cu") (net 7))
 (segment (start 166.46 60) (end 164.27 62.19) (width 0.2) (layer "B.Cu") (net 7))
 (segment (start 194 65.938) (end 194 66) (width 0.2) (layer "B.Cu") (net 7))
 (segment (start 193.962942 66) (end 184.962942 75) (width 0.2) (layer "B.Cu") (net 7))
 (segment (start 184.962942 75) (end 180 75) (width 0.2) (layer "B.Cu") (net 7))
 (segment (start 168 63) (end 168 61.54) (width 0.2) (layer "B.Cu") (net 7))
 (segment (start 164.27 64.73) (end 140 64.73) (width 0.2) (layer "F.Cu") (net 8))
 (segment (start 169 60) (end 164.27 64.73) (width 0.2) (layer "F.Cu") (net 8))
 (segment (start 195.676 65.074) (end 195.676 69.317058) (width 0.2) (layer "B.Cu") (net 8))
 (segment (start 185.949 75.949) (end 179.759936 75.949) (width 0.2) (layer "B.Cu") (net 8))
 (segment (start 186 76) (end 185.949 75.949) (width 0.2) (layer "B.Cu") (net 8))
 (segment (start 179.759936 75.949) (end 169 65.189064) (width 0.2) (layer "B.Cu") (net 8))
 (segment (start 169 65.189064) (end 169 60) (width 0.2) (layer "B.Cu") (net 8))
 (segment (start 194 63.398) (end 195.676 65.074) (width 0.2) (layer "B.Cu") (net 8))
 (segment (start 188.993058 76) (end 186 76) (width 0.2) (layer "B.Cu") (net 8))
 (segment (start 195.676 69.317058) (end 188.993058 76) (width 0.2) (layer "B.Cu") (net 8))
 (segment (start 163.92 62.92) (end 164 63) (width 0.2) (layer "F.Cu") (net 2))
 (segment (start 172 58) (end 163 58) (width 0.2) (layer "F.Cu") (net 2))
 (segment (start 163.92 60) (end 163 59.08) (width 0.2) (layer "F.Cu") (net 2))
 (segment (start 139.35 59) (end 137 59) (width 0.2) (layer "F.Cu") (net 2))
 (segment (start 163.92 60) (end 163.92 62.92) (width 0.2) (layer "F.Cu") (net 2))
 (segment (start 175.182765 54.817235) (end 172 58) (width 0.2) (layer "F.Cu") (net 2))
 (segment (start 163 59.08) (end 163 58) (width 0.2) (layer "F.Cu") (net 2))
 (segment (start 140 59.65) (end 139.35 59) (width 0.2) (layer "F.Cu") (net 2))
 (via (at 164 63) (size 0.6) (drill 0.3) (layers "F.Cu" "B.Cu") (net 2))
 (via (at 163 58) (size 0.6) (drill 0.3) (layers "F.Cu" "B.Cu") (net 2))
 (via (at 137 59) (size 0.6) (drill 0.3) (layers "F.Cu" "B.Cu") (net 2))
 (via (at 175.182765 54.817235) (size 0.6) (drill 0.3) (layers "F.Cu" "B.Cu") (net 2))
 (segment (start 140.047157 94.6) (end 139.599999 94.152842) (width 0.2) (layer "B.Cu") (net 2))
 (segment (start 139.599999 94.352842) (end 139.599999 93.6) (width 0.2) (layer "B.Cu") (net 2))
 (segment (start 139.599999 93.6) (end 139.599999 92.117759) (width 0.2) (layer "B.Cu") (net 2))
 (segment (start 148.38 102.38) (end 148.38 114.92) (width 0.2) (layer "B.Cu") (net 2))
 (segment (start 167.599999 115.079999) (end 167.44 114.92) (width 0.2) (layer "B.Cu") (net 2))
 (segment (start 163 58) (end 162.400001 57.400001) (width 0.2) (layer "B.Cu") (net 2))
 (segment (start 167.599999 134.352842) (end 167.599999 115.079999) (width 0.2) (layer "B.Cu") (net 2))
 (segment (start 162.400001 57.400001) (end 142.249999 57.400001) (width 0.2) (layer "B.Cu") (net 2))
 (segment (start 176.14353 55.778) (end 175.182765 54.817235) (width 0.2) (layer "B.Cu") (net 2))
 (segment (start 139.599999 92.117759) (end 139.48224 92) (width 0.2) (layer "B.Cu") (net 2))
 (segment (start 135 92) (end 135 58.775) (width 0.2) (layer "B.Cu") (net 2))
 (segment (start 167.44 114.92) (end 148.38 114.92) (width 0.2) (layer "B.Cu") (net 2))
 (segment (start 140.6 94.6) (end 148.38 102.38) (width 0.2) (layer "B.Cu") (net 2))
 (segment (start 139.48224 92) (end 135 92) (width 0.2) (layer "B.Cu") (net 2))
 (segment (start 139.599999 94.352842) (end 140.352842 94.352842) (width 0.2) (layer "B.Cu") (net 2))
 (segment (start 162.400001 57.400001) (end 162.400001 55.96) (width 0.2) (layer "B.Cu") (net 2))
 (segment (start 177.835 55.778) (end 176.14353 55.778) (width 0.2) (layer "B.Cu") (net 2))
 (segment (start 140.352842 94.352842) (end 140.6 94.6) (width 0.2) (layer "B.Cu") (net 2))
 (segment (start 142.249999 57.400001) (end 140 59.65) (width 0.2) (layer "B.Cu") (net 2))
 (segment (start 136.775 58.775) (end 135 58.775) (width 0.2) (layer "B.Cu") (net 2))
 (segment (start 186.49 114.92) (end 167.44 114.92) (width 0.2) (layer "B.Cu") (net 2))
 (segment (start 191.45 109.96) (end 186.49 114.92) (width 0.2) (layer "B.Cu") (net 2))
 (segment (start 190.400001 102.950001) (end 190.400001 95.647158) (width 0.2) (layer "B.Cu") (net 2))
 (segment (start 137 59) (end 136.775 58.775) (width 0.2) (layer "B.Cu") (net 2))
 (segment (start 139.599999 93.6) (end 139.599999 94.152842) (width 0.2) (layer "B.Cu") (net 2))
 (segment (start 191.45 104) (end 191.45 109.96) (width 0.2) (layer "B.Cu") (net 2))
 (segment (start 140.6 94.6) (end 140.047157 94.6) (width 0.2) (layer "B.Cu") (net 2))
 (segment (start 191.45 104) (end 190.400001 102.950001) (width 0.2) (layer "B.Cu") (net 2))
 (segment (start 164 63) (end 164 64) (width 0.2) (layer "B.Cu") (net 2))
 (segment (start 151 109) (end 150.49 109) (width 0.2) (layer "F.Cu") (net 5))
 (segment (start 150.49 109) (end 142.03 117.46) (width 0.2) (layer "F.Cu") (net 5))
 (via (at 151 109) (size 0.6) (drill 0.3) (layers "F.Cu" "B.Cu") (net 5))
 (segment (start 196.879 56.117) (end 196.879 78.538043) (width 0.2) (layer "B.Cu") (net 5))
 (segment (start 194 53.238) (end 196.879 56.117) (width 0.2) (layer "B.Cu") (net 5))
 (segment (start 196.879 78.538043) (end 166.417043 109) (width 0.2) (layer "B.Cu") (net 5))
 (segment (start 166.417043 109) (end 151 109) (width 0.2) (layer "B.Cu") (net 5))
 (segment (start 161 104) (end 161.09 104.09) (width 0.2) (layer "F.Cu") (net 9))
 (segment (start 161.09 104.09) (end 161.09 117.46) (width 0.2) (layer "F.Cu") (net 9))
 (segment (start 161 103) (end 161 104) (width 0.2) (layer "F.Cu") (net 9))
 (via (at 161 103) (size 0.6) (drill 0.3) (layers "F.Cu" "B.Cu") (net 9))
 (segment (start 196.478 58.256) (end 196.478 78.371943) (width 0.2) (layer "B.Cu") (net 9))
 (segment (start 171.849943 103) (end 161 103) (width 0.2) (layer "B.Cu") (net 9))
 (segment (start 194 55.778) (end 196.478 58.256) (width 0.2) (layer "B.Cu") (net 9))
 (segment (start 196.478 78.371943) (end 171.849943 103) (width 0.2) (layer "B.Cu") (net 9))
 (segment (start 180.14 94.86) (end 180.14 117.46) (width 0.2) (layer "F.Cu") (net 6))
 (segment (start 181 93) (end 181 94) (width 0.2) (layer "F.Cu") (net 6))
 (segment (start 181 94) (end 180.14 94.86) (width 0.2) (layer "F.Cu") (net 6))
 (via (at 181 93) (size 0.6) (drill 0.3) (layers "F.Cu" "B.Cu") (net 6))
 (segment (start 194 58.318) (end 196.077 60.395) (width 0.2) (layer "B.Cu") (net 6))
 (segment (start 196.077 60.395) (end 196.077 77.923) (width 0.2) (layer "B.Cu") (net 6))
 (segment (start 196.077 77.923) (end 181 93) (width 0.2) (layer "B.Cu") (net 6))
 (segment (start 134 58) (end 134 92) (width 0.2) (layer "F.Cu") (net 4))
 (segment (start 161.38 60) (end 161.38 62.38) (width 0.2) (layer "F.Cu") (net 4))
 (segment (start 161.38 60) (end 142.89 60) (width 0.2) (layer "F.Cu") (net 4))
 (segment (start 194 104) (end 197 104) (width 0.2) (layer "F.Cu") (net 4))
 (segment (start 194 104) (end 194 113.33153) (width 0.2) (layer "F.Cu") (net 4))
 (segment (start 142.89 60) (end 140 57.11) (width 0.2) (layer "F.Cu") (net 4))
 (segment (start 194 113.33153) (end 168.33153 139) (width 0.2) (layer "F.Cu") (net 4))
 (segment (start 140 57.11) (end 134.89 57.11) (width 0.2) (layer "F.Cu") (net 4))
 (segment (start 168.33153 139) (end 166 139) (width 0.2) (layer "F.Cu") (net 4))
 (segment (start 161.38 62.38) (end 162 63) (width 0.2) (layer "F.Cu") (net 4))
 (segment (start 134 92) (end 132 94) (width 0.2) (layer "F.Cu") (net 4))
 (segment (start 161.38 60) (end 162 59.38) (width 0.2) (layer "F.Cu") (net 4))
 (segment (start 134.89 57.11) (end 134 58) (width 0.2) (layer "F.Cu") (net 4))
 (segment (start 162 59.38) (end 162 53) (width 0.2) (layer "F.Cu") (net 4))
 (via (at 132 94) (size 0.6) (drill 0.3) (layers "F.Cu" "B.Cu") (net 4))
 (via (at 134 58) (size 0.6) (drill 0.3) (layers "F.Cu" "B.Cu") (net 4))
 (via (at 166 139) (size 0.6) (drill 0.3) (layers "F.Cu" "B.Cu") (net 4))
 (via (at 162 53) (size 0.6) (drill 0.3) (layers "F.Cu" "B.Cu") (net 4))
 (via (at 194 104) (size 0.6) (drill 0.3) (layers "F.Cu" "B.Cu") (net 4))
 (via (at 162 63) (size 0.6) (drill 0.3) (layers "F.Cu" "B.Cu") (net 4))
 (via (at 197 104) (size 0.6) (drill 0.3) (layers "F.Cu" "B.Cu") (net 4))
 (segment (start 134.775 57.225) (end 134 58) (width 0.2) (layer "B.Cu") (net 4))
 (segment (start 166 52) (end 163 52) (width 0.2) (layer "B.Cu") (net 4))
 (segment (start 160 135.852842) (end 162.399999 135.852842) (width 0.2) (layer "B.Cu") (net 4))
 (segment (start 195.600001 94.147158) (end 195.689915 94.147158) (width 0.2) (layer "B.Cu") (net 4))
 (segment (start 180 76.65) (end 175.1 76.65) (width 0.2) (layer "B.Cu") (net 4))
 (segment (start 177.835 58.318) (end 173.977 54.46) (width 0.2) (layer "B.Cu") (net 4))
 (segment (start 177.835 58.165) (end 178 58) (width 0.2) (layer "B.Cu") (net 4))
 (segment (start 167.600001 53.600001) (end 166 52) (width 0.2) (layer "B.Cu") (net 4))
 (segment (start 167.600001 54.46) (end 167.600001 53.600001) (width 0.2) (layer "B.Cu") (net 4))
 (segment (start 195.689915 94.147158) (end 197 95.457243) (width 0.2) (layer "B.Cu") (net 4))
 (segment (start 163 52) (end 162 53) (width 0.2) (layer "B.Cu") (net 4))
 (segment (start 186 77.65) (end 181 77.65) (width 0.2) (layer "B.Cu") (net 4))
 (segment (start 134.399999 95.852842) (end 134.399999 133.967099) (width 0.2) (layer "B.Cu") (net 4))
 (segment (start 133.852842 95.852842) (end 134.399999 95.852842) (width 0.2) (layer "B.Cu") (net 4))
 (segment (start 175.1 76.65) (end 162.45 64) (width 0.2) (layer "B.Cu") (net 4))
 (segment (start 132 94) (end 133.852842 95.852842) (width 0.2) (layer "B.Cu") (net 4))
 (segment (start 162 63) (end 162 63.55) (width 0.2) (layer "B.Cu") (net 4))
 (segment (start 162 63.55) (end 162.45 64) (width 0.2) (layer "B.Cu") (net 4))
 (segment (start 134.399999 133.967099) (end 136.285742 135.852842) (width 0.2) (layer "B.Cu") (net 4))
 (segment (start 193 104) (end 194 104) (width 0.2) (layer "B.Cu") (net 4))
 (segment (start 166 139) (end 163.147158 139) (width 0.2) (layer "B.Cu") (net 4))
 (segment (start 173.977 54.46) (end 167.600001 54.46) (width 0.2) (layer "B.Cu") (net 4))
 (segment (start 181 77.65) (end 180 76.65) (width 0.2) (layer "B.Cu") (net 4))
 (segment (start 197 95.457243) (end 197 104) (width 0.2) (layer "B.Cu") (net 4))
 (segment (start 163.147158 139) (end 160 135.852842) (width 0.2) (layer "B.Cu") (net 4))
 (segment (start 136.285742 135.852842) (end 160 135.852842) (width 0.2) (layer "B.Cu") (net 4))
 (segment (start 135 57.225) (end 134.775 57.225) (width 0.2) (layer "B.Cu") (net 4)))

